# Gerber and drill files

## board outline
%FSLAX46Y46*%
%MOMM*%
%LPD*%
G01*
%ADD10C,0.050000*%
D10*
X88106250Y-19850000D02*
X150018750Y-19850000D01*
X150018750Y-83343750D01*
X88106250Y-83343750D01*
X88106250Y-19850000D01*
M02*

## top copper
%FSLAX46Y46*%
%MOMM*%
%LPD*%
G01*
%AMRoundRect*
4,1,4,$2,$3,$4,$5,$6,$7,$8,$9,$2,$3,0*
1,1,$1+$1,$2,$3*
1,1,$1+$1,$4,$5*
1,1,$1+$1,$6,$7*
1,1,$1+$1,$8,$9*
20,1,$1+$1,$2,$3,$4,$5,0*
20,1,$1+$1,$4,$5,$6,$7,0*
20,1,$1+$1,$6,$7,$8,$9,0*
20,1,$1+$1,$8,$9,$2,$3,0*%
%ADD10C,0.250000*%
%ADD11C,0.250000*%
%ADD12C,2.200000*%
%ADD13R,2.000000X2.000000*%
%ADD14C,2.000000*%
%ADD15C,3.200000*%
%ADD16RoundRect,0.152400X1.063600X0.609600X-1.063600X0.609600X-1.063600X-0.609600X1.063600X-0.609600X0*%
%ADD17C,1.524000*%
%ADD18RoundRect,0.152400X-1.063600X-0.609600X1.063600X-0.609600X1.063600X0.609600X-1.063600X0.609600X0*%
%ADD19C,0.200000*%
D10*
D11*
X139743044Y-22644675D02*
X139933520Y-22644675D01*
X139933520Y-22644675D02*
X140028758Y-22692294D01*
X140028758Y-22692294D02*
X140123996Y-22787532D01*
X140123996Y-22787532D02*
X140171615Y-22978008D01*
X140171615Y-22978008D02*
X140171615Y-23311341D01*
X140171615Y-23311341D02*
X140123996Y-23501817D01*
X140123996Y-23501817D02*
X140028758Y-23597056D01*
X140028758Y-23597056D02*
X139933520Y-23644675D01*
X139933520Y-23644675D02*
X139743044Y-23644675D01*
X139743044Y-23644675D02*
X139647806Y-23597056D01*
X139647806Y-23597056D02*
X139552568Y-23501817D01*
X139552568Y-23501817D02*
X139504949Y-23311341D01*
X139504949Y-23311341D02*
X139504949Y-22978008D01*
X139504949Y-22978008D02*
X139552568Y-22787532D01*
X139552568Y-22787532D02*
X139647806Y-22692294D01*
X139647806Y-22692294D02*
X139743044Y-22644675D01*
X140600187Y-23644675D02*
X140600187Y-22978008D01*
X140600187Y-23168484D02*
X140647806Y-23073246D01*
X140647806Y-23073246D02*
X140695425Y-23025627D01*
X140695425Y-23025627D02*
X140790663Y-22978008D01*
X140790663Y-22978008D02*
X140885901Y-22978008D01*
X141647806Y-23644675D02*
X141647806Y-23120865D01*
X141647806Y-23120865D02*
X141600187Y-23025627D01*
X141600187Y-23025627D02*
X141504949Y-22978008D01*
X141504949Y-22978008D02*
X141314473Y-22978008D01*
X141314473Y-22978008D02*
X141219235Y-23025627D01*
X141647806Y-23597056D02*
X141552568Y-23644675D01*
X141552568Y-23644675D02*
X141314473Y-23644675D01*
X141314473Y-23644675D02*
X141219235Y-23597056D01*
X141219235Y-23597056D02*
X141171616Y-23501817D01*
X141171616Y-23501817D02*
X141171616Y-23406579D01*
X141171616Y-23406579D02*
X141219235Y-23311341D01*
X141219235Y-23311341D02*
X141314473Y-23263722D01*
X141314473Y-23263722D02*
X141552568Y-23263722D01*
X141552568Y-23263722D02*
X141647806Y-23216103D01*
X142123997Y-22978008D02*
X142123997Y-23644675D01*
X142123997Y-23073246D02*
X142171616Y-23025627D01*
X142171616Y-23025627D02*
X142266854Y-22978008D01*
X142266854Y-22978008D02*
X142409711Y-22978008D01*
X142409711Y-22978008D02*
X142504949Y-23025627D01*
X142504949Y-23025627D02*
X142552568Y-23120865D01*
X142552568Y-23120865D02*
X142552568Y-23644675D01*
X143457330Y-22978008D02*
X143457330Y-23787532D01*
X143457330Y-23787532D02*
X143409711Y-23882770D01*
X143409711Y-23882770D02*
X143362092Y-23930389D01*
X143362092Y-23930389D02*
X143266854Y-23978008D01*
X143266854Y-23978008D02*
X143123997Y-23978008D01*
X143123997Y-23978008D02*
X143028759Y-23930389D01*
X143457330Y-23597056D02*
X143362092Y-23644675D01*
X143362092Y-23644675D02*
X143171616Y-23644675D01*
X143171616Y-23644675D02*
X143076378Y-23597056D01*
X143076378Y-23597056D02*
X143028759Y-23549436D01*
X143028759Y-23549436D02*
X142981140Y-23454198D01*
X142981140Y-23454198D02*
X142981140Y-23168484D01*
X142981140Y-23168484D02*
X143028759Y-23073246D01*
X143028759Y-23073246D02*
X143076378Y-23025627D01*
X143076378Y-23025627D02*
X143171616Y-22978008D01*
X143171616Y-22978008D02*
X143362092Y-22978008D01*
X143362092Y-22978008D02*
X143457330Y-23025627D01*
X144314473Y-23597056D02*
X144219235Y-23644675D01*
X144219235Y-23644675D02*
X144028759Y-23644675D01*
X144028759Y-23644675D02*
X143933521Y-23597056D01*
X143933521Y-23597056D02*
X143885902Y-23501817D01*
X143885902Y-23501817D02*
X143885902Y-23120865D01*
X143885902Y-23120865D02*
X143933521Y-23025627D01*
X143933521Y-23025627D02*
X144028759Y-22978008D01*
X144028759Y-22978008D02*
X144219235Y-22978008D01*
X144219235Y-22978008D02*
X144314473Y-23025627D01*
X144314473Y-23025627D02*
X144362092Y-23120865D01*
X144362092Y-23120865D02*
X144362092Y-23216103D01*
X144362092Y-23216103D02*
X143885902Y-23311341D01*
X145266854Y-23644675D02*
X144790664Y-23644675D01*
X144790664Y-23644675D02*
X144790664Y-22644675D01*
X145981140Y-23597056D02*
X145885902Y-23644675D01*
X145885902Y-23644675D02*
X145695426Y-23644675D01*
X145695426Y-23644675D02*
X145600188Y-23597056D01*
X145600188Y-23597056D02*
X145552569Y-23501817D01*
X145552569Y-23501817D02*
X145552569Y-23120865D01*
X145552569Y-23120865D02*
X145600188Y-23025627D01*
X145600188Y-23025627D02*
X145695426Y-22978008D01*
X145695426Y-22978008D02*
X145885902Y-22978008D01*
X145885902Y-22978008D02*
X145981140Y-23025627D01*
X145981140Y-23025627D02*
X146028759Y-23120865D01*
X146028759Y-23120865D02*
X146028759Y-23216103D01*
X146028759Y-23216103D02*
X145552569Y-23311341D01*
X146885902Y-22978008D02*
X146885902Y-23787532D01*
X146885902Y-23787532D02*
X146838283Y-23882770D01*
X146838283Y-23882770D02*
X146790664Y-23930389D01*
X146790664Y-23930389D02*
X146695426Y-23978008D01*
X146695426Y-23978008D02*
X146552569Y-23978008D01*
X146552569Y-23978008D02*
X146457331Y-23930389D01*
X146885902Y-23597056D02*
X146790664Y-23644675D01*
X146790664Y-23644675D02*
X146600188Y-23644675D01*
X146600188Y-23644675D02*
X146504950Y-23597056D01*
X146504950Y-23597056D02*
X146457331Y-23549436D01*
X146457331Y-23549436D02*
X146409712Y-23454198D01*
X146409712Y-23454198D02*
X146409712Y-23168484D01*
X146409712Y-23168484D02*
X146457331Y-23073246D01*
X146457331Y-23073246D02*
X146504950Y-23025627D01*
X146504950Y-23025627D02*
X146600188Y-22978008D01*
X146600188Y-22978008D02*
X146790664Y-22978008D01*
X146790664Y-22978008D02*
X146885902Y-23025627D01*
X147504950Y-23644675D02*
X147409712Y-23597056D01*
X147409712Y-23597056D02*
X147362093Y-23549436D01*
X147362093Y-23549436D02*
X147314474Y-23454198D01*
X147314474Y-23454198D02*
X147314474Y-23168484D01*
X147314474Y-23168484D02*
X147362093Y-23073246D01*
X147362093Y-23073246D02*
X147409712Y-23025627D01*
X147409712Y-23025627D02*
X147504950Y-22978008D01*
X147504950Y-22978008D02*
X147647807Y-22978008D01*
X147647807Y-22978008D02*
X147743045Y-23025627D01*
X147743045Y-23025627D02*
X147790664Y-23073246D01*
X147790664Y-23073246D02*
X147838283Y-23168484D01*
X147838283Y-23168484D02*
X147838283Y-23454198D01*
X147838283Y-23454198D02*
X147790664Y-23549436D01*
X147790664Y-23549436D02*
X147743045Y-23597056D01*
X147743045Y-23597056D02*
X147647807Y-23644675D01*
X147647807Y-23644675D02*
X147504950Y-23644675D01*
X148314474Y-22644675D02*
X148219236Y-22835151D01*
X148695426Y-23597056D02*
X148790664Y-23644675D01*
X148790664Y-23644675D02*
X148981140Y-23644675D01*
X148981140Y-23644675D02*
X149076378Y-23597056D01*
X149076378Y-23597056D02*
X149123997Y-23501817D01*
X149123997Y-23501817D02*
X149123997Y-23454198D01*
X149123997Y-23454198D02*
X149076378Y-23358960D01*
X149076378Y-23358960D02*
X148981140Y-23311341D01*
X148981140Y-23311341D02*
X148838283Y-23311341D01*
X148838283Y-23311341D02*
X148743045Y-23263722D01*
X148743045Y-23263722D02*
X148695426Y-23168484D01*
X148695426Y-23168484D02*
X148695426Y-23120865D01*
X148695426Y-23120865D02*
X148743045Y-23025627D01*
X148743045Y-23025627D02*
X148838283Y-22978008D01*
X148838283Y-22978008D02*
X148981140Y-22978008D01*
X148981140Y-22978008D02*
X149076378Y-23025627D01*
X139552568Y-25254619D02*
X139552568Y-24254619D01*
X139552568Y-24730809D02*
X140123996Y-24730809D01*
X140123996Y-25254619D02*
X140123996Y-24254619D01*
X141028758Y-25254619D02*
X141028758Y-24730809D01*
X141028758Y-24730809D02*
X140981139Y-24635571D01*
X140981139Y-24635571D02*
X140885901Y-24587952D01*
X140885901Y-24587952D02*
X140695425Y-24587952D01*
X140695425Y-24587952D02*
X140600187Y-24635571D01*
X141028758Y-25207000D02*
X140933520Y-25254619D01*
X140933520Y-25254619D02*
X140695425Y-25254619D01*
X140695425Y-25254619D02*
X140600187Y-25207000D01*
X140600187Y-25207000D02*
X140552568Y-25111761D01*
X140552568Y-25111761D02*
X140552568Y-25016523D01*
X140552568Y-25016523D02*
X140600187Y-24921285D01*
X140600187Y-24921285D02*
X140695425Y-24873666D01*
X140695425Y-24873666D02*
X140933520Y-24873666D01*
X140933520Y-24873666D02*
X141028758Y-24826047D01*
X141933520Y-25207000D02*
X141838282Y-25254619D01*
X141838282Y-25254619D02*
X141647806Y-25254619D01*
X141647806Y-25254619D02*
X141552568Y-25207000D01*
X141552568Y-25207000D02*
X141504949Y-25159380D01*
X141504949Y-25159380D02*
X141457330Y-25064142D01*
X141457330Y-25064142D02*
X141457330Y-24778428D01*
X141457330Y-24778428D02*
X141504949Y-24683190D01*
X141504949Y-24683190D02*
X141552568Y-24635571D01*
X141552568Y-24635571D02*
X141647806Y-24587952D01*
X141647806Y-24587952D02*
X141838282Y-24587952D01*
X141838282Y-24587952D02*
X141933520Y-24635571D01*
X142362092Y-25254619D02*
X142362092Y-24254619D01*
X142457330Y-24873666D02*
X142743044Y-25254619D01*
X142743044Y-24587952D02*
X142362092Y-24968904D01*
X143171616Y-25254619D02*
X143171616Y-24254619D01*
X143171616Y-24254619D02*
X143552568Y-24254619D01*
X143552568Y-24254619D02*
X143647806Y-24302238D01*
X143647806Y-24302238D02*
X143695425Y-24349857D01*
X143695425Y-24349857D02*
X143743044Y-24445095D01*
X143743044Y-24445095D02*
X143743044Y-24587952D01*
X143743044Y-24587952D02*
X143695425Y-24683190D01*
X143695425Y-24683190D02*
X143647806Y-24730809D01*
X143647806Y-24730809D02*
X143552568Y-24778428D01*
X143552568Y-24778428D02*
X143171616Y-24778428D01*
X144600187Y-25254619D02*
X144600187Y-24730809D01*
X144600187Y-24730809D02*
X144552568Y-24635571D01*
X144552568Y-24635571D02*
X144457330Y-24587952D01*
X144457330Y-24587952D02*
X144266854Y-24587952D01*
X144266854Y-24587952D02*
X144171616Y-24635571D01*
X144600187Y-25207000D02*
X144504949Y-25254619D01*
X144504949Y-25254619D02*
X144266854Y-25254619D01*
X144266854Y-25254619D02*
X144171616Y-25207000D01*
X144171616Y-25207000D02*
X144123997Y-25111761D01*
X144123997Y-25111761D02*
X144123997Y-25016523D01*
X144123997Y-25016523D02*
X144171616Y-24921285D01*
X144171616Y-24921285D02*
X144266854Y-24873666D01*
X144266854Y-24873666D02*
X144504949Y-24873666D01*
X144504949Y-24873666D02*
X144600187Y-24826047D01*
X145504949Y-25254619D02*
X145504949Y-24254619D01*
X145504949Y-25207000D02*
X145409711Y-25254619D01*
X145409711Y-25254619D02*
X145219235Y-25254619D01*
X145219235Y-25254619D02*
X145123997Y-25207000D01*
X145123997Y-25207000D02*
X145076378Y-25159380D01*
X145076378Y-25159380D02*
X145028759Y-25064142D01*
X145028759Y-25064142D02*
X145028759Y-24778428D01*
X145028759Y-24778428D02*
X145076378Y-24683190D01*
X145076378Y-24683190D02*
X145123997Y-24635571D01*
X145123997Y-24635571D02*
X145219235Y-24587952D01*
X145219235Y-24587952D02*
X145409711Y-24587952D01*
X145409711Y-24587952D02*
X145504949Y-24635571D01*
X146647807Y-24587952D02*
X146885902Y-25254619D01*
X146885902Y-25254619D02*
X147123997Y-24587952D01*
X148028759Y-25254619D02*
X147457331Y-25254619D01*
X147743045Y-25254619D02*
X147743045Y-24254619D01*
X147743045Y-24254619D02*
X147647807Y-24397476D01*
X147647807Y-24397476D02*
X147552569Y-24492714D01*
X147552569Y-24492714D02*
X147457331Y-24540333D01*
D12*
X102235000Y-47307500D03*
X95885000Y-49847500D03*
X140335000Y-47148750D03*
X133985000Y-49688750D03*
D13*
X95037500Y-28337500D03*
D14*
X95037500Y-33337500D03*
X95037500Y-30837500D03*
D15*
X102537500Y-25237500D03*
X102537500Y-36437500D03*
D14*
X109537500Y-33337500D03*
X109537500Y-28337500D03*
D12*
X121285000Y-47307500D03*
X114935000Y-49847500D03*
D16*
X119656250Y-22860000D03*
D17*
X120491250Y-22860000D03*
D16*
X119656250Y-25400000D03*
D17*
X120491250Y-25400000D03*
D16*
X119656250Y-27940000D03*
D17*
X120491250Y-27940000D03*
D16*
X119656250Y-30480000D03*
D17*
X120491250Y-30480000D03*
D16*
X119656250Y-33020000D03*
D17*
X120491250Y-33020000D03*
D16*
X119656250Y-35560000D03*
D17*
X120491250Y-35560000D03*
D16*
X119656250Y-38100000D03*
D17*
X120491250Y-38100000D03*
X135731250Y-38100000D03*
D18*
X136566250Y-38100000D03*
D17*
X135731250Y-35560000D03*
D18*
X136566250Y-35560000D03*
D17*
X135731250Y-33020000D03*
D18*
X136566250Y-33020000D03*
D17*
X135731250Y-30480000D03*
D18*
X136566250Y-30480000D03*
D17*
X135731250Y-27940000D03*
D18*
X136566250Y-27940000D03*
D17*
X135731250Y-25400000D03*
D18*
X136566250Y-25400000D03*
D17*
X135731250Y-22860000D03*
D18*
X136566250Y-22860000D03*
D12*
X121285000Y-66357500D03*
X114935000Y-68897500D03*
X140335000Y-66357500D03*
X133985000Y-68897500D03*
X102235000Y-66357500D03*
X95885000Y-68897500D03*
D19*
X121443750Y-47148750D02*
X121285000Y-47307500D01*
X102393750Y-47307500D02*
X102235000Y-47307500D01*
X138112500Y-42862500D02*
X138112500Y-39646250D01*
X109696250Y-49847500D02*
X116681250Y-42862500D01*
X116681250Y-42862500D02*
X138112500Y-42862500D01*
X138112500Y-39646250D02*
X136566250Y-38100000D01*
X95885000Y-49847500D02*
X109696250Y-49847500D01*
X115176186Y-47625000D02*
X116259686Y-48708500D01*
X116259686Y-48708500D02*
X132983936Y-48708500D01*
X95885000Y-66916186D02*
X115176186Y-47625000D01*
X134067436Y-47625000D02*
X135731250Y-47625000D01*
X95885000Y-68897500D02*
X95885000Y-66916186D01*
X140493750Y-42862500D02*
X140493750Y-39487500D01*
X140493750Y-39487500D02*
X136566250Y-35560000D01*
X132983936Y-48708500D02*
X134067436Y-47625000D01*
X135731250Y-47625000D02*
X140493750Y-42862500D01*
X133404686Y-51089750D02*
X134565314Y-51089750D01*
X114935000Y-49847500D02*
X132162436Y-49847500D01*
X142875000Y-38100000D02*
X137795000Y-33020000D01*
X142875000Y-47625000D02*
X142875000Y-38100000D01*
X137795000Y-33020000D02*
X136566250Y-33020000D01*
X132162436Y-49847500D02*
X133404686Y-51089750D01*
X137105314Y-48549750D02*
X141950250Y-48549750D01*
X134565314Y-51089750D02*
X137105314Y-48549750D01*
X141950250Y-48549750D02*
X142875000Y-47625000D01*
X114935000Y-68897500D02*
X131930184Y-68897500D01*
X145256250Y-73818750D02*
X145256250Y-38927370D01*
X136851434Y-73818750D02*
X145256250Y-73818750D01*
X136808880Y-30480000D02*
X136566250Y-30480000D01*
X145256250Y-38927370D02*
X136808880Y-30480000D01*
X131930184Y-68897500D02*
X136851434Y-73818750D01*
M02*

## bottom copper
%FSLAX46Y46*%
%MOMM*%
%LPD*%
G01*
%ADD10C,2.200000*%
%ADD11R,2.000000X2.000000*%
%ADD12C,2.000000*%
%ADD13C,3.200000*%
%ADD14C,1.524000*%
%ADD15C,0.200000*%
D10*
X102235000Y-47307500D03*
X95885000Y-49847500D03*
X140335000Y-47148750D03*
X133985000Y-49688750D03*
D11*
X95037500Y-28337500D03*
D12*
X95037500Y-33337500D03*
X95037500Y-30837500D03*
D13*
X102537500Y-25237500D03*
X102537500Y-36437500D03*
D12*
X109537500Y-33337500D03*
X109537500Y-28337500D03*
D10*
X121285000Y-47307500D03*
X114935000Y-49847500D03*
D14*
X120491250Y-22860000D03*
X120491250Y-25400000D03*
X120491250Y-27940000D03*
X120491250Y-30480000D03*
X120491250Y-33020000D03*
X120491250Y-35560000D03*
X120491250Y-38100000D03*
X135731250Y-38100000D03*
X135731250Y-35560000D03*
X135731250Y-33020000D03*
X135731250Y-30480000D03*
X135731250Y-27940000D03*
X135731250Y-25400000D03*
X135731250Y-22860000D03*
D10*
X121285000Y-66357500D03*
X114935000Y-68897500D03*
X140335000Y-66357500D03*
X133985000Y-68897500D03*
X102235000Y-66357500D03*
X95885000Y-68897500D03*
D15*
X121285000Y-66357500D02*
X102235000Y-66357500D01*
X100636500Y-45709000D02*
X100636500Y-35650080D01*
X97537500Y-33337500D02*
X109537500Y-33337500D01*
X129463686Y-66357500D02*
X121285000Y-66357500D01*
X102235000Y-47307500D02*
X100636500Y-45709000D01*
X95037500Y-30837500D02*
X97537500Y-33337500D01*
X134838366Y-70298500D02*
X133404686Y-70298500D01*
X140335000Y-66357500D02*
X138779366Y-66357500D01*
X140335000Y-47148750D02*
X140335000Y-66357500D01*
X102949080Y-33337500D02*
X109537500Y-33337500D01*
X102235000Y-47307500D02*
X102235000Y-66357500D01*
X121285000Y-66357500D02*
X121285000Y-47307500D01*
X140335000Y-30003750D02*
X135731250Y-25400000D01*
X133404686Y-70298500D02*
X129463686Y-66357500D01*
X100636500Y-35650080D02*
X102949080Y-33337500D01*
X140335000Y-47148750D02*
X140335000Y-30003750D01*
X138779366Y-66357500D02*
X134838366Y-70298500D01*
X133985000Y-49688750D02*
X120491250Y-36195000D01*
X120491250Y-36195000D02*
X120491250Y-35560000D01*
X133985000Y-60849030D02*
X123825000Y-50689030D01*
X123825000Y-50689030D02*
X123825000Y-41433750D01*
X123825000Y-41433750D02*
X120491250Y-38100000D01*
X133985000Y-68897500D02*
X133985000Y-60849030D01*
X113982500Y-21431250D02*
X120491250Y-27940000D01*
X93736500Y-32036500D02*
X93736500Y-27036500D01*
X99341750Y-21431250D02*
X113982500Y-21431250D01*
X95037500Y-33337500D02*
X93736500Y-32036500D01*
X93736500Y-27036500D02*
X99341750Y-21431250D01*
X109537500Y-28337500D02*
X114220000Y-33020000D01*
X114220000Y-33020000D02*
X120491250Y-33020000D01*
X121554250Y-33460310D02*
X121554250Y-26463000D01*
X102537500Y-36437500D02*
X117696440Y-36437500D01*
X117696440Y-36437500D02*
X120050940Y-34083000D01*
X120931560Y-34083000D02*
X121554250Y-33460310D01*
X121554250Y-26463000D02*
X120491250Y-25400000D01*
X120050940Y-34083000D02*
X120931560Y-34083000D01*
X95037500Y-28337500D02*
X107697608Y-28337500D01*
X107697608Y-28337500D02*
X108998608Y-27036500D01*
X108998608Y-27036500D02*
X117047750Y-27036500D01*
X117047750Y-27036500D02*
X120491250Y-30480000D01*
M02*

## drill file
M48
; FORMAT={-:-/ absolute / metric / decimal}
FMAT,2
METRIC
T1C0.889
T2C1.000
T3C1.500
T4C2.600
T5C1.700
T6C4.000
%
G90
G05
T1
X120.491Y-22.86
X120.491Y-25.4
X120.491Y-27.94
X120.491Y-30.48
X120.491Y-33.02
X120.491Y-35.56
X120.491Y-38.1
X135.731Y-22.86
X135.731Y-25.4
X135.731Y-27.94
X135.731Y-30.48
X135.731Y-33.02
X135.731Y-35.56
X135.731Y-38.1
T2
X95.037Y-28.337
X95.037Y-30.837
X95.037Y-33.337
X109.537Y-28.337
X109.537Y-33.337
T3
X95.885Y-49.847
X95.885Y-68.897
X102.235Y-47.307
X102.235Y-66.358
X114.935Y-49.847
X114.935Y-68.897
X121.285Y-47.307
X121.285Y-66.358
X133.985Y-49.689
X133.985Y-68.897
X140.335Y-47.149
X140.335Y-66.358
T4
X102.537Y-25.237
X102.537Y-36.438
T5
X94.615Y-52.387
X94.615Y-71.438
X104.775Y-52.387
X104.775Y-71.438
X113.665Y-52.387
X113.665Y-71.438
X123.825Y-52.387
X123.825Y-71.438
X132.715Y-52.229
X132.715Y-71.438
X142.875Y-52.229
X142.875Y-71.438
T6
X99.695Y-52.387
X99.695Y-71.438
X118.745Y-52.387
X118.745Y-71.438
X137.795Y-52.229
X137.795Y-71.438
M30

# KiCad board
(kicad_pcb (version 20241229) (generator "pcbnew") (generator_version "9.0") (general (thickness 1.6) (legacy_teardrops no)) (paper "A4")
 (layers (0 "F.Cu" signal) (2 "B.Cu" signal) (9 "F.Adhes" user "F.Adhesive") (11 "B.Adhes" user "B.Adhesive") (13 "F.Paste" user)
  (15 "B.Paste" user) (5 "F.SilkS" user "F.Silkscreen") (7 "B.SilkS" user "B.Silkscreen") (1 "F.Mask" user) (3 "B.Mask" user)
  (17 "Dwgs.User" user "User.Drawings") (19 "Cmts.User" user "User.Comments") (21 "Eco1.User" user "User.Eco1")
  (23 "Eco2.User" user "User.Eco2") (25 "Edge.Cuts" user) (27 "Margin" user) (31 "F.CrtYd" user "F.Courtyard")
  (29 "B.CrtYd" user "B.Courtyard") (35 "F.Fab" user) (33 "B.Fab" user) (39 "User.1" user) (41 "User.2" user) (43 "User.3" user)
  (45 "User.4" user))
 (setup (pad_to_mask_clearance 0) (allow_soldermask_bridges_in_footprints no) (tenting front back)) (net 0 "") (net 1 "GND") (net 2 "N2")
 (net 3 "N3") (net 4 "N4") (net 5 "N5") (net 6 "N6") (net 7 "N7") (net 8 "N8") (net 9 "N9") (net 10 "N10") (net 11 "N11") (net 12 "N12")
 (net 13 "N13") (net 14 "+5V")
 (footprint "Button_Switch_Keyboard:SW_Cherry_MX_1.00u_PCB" (layer "F.Cu") (at 102.235 47.3075)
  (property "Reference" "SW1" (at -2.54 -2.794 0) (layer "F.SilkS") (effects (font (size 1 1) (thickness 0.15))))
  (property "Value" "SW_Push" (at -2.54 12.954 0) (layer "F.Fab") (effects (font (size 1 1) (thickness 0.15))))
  (pad "" np_thru_hole circle (at -7.62 5.08) (size 1.7 1.7) (drill 1.7) (layers "*.Cu" "*.Mask"))
  (pad "" np_thru_hole circle (at -2.54 5.08) (size 4 4) (drill 4) (layers "*.Cu" "*.Mask"))
  (pad "" np_thru_hole circle (at 2.54 5.08) (size 1.7 1.7) (drill 1.7) (layers "*.Cu" "*.Mask"))
  (pad "1" thru_hole circle (at 0 0) (size 2.2 2.2) (drill 1.5) (layers "*.Cu" "*.Mask") (remove_unused_layers no) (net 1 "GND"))
  (pad "2" thru_hole circle (at -6.35 2.54) (size 2.2 2.2) (drill 1.5) (layers "*.Cu" "*.Mask") (remove_unused_layers no) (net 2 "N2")))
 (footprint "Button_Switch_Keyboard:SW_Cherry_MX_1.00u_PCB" (layer "F.Cu") (at 140.335 47.14875)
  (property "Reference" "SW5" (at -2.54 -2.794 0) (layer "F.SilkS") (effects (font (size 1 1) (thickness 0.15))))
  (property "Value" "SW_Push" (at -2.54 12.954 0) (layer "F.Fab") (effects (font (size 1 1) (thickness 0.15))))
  (pad "" np_thru_hole circle (at -7.62 5.08) (size 1.7 1.7) (drill 1.7) (layers "*.Cu" "*.Mask"))
  (pad "" np_thru_hole circle (at -2.54 5.08) (size 4 4) (drill 4) (layers "*.Cu" "*.Mask"))
  (pad "" np_thru_hole circle (at 2.54 5.08) (size 1.7 1.7) (drill 1.7) (layers "*.Cu" "*.Mask"))
  (pad "1" thru_hole circle (at 0 0) (size 2.2 2.2) (drill 1.5) (layers "*.Cu" "*.Mask") (remove_unused_layers no) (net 1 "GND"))
  (pad "2" thru_hole circle (at -6.35 2.54) (size 2.2 2.2) (drill 1.5) (layers "*.Cu" "*.Mask") (remove_unused_layers no) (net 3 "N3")))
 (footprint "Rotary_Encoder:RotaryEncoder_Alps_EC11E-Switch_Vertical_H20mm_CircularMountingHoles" (layer "F.Cu") (at 95.0375 28.3375)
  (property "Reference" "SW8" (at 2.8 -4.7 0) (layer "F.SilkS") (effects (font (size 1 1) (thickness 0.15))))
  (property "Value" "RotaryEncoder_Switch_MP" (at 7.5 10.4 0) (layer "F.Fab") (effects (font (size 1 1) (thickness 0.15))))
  (pad "A" thru_hole rect (at 0 0) (size 2 2) (drill 1) (layers "*.Cu" "*.Mask") (remove_unused_layers no) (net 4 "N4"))
  (pad "B" thru_hole circle (at 0 5) (size 2 2) (drill 1) (layers "*.Cu" "*.Mask") (remove_unused_layers no) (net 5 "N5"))
  (pad "C" thru_hole circle (at 0 2.5) (size 2 2) (drill 1) (layers "*.Cu" "*.Mask") (remove_unused_layers no) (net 1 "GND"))
  (pad "MP" thru_hole circle (at 7.5 -3.1) (size 3.2 3.2) (drill 2.6) (layers "*.Cu" "*.Mask") (remove_unused_layers no) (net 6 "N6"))
  (pad "MP" thru_hole circle (at 7.5 8.1) (size 3.2 3.2) (drill 2.6) (layers "*.Cu" "*.Mask") (remove_unused_layers no) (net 6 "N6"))
  (pad "S1" thru_hole circle (at 14.5 5) (size 2 2) (drill 1) (layers "*.Cu" "*.Mask") (remove_unused_layers no) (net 1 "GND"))
  (pad "S2" thru_hole circle (at 14.5 0) (size 2 2) (drill 1) (layers "*.Cu" "*.Mask") (remove_unused_layers no) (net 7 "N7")))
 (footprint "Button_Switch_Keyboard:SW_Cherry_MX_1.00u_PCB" (layer "F.Cu") (at 121.285 47.3075)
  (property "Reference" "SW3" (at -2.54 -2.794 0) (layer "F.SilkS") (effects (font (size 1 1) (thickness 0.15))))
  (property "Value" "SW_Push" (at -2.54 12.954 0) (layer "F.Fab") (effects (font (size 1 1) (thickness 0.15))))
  (pad "" np_thru_hole circle (at -7.62 5.08) (size 1.7 1.7) (drill 1.7) (layers "*.Cu" "*.Mask"))
  (pad "" np_thru_hole circle (at -2.54 5.08) (size 4 4) (drill 4) (layers "*.Cu" "*.Mask"))
  (pad "" np_thru_hole circle (at 2.54 5.08) (size 1.7 1.7) (drill 1.7) (layers "*.Cu" "*.Mask"))
  (pad "1" thru_hole circle (at 0 0) (size 2.2 2.2) (drill 1.5) (layers "*.Cu" "*.Mask") (remove_unused_layers no) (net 1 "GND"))
  (pad "2" thru_hole circle (at -6.35 2.54) (size 2.2 2.2) (drill 1.5) (layers "*.Cu" "*.Mask") (remove_unused_layers no) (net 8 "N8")))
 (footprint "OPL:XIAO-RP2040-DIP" (layer "F.Cu") (at 128.11125 30.48)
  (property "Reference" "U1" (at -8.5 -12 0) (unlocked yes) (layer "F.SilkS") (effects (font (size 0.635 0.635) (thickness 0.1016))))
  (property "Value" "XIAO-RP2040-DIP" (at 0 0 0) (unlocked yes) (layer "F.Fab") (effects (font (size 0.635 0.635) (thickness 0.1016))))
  (pad "1" smd roundrect (at -8.455 -7.62 180) (size 2.432 1.524) (layers "F.Cu" "F.Mask") (roundrect_rratio 0.1) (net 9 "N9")
   (thermal_bridge_angle 45))
  (pad "1" thru_hole circle (at -7.62 -7.62 180) (size 1.524 1.524) (drill 0.889) (layers "*.Cu" "*.Mask") (remove_unused_layers no)
   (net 9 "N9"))
  (pad "2" smd roundrect (at -8.455 -5.08 180) (size 2.432 1.524) (layers "F.Cu" "F.Mask") (roundrect_rratio 0.1) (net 6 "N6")
   (thermal_bridge_angle 45))
  (pad "2" thru_hole circle (at -7.62 -5.08 180) (size 1.524 1.524) (drill 0.889) (layers "*.Cu" "*.Mask") (remove_unused_layers no)
   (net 6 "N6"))
  (pad "3" smd roundrect (at -8.455 -2.54 180) (size 2.432 1.524) (layers "F.Cu" "F.Mask") (roundrect_rratio 0.1) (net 5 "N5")
   (thermal_bridge_angle 45))
  (pad "3" thru_hole circle (at -7.62 -2.54 180) (size 1.524 1.524) (drill 0.889) (layers "*.Cu" "*.Mask") (remove_unused_layers no)
   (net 5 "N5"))
  (pad "4" smd roundrect (at -8.455 0 180) (size 2.432 1.524) (layers "F.Cu" "F.Mask") (roundrect_rratio 0.1) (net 4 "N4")
   (thermal_bridge_angle 45))
  (pad "4" thru_hole circle (at -7.62 0 180) (size 1.524 1.524) (drill 0.889) (layers "*.Cu" "*.Mask") (remove_unused_layers no)
   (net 4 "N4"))
  (pad "5" smd roundrect (at -8.455 2.54 180) (size 2.432 1.524) (layers "F.Cu" "F.Mask") (roundrect_rratio 0.1) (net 7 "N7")
   (thermal_bridge_angle 45))
  (pad "5" thru_hole circle (at -7.62 2.54 180) (size 1.524 1.524) (drill 0.889) (layers "*.Cu" "*.Mask") (remove_unused_layers no)
   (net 7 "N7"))
  (pad "6" smd roundrect (at -8.455 5.08 180) (size 2.432 1.524) (layers "F.Cu" "F.Mask") (roundrect_rratio 0.1) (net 3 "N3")
   (thermal_bridge_angle 45))
  (pad "6" thru_hole circle (at -7.62 5.08 180) (size 1.524 1.524) (drill 0.889) (layers "*.Cu" "*.Mask") (remove_unused_layers no)
   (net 3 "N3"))
  (pad "7" smd roundrect (at -8.455 7.62 180) (size 2.432 1.524) (layers "F.Cu" "F.Mask") (roundrect_rratio 0.1) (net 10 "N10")
   (thermal_bridge_angle 45))
  (pad "7" thru_hole circle (at -7.62 7.62 180) (size 1.524 1.524) (drill 0.889) (layers "*.Cu" "*.Mask") (remove_unused_layers no)
   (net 10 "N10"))
  (pad "8" thru_hole circle (at 7.62 7.62) (size 1.524 1.524) (drill 0.889) (layers "*.Cu" "*.Mask") (remove_unused_layers no) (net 2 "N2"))
  (pad "8" smd roundrect (at 8.455 7.62) (size 2.432 1.524) (layers "F.Cu" "F.Mask") (roundrect_rratio 0.1) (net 2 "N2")
   (thermal_bridge_angle 45))
  (pad "9" thru_hole circle (at 7.62 5.08) (size 1.524 1.524) (drill 0.889) (layers "*.Cu" "*.Mask") (remove_unused_layers no)
   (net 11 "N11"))
  (pad "9" smd roundrect (at 8.455 5.08) (size 2.432 1.524) (layers "F.Cu" "F.Mask") (roundrect_rratio 0.1) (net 11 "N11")
   (thermal_bridge_angle 45))
  (pad "10" thru_hole circle (at 7.62 2.54) (size 1.524 1.524) (drill 0.889) (layers "*.Cu" "*.Mask") (remove_unused_layers no) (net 8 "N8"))
  (pad "10" smd roundrect (at 8.455 2.54) (size 2.432 1.524) (layers "F.Cu" "F.Mask") (roundrect_rratio 0.1) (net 8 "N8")
   (thermal_bridge_angle 45))
  (pad "11" thru_hole circle (at 7.62 0) (size 1.524 1.524) (drill 0.889) (layers "*.Cu" "*.Mask") (remove_unused_layers no) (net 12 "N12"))
  (pad "11" smd roundrect (at 8.455 0) (size 2.432 1.524) (layers "F.Cu" "F.Mask") (roundrect_rratio 0.1) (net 12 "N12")
   (thermal_bridge_angle 45))
  (pad "12" thru_hole circle (at 7.62 -2.54) (size 1.524 1.524) (drill 0.889) (layers "*.Cu" "*.Mask") (remove_unused_layers no)
   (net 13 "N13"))
  (pad "12" smd roundrect (at 8.455 -2.54) (size 2.432 1.524) (layers "F.Cu" "F.Mask") (roundrect_rratio 0.1) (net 13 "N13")
   (thermal_bridge_angle 45))
  (pad "13" thru_hole circle (at 7.62 -5.08) (size 1.524 1.524) (drill 0.889) (layers "*.Cu" "*.Mask") (remove_unused_layers no)
   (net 1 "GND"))
  (pad "13" smd roundrect (at 8.455 -5.08) (size 2.432 1.524) (layers "F.Cu" "F.Mask") (roundrect_rratio 0.1) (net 1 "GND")
   (thermal_bridge_angle 45))
  (pad "14" thru_hole circle (at 7.62 -7.62) (size 1.524 1.524) (drill 0.889) (layers "*.Cu" "*.Mask") (remove_unused_layers no)
   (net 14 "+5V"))
  (pad "14" smd roundrect (at 8.455 -7.62) (size 2.432 1.524) (layers "F.Cu" "F.Mask") (roundrect_rratio 0.1) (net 14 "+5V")
   (thermal_bridge_angle 45)))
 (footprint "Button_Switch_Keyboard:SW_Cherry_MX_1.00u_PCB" (layer "F.Cu") (at 121.285 66.3575)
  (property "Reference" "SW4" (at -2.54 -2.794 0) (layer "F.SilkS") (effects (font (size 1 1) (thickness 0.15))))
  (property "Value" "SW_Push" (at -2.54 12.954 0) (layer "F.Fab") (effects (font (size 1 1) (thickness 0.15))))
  (pad "" np_thru_hole circle (at -7.62 5.08) (size 1.7 1.7) (drill 1.7) (layers "*.Cu" "*.Mask"))
  (pad "" np_thru_hole circle (at -2.54 5.08) (size 4 4) (drill 4) (layers "*.Cu" "*.Mask"))
  (pad "" np_thru_hole circle (at 2.54 5.08) (size 1.7 1.7) (drill 1.7) (layers "*.Cu" "*.Mask"))
  (pad "1" thru_hole circle (at 0 0) (size 2.2 2.2) (drill 1.5) (layers "*.Cu" "*.Mask") (remove_unused_layers no) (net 1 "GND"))
  (pad "2" thru_hole circle (at -6.35 2.54) (size 2.2 2.2) (drill 1.5) (layers "*.Cu" "*.Mask") (remove_unused_layers no) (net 12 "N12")))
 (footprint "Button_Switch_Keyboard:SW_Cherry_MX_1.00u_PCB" (layer "F.Cu") (at 140.335 66.3575)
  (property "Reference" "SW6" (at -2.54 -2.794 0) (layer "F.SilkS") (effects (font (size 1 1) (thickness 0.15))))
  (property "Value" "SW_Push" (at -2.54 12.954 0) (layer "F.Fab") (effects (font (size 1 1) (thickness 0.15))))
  (pad "" np_thru_hole circle (at -7.62 5.08) (size 1.7 1.7) (drill 1.7) (layers "*.Cu" "*.Mask"))
  (pad "" np_thru_hole circle (at -2.54 5.08) (size 4 4) (drill 4) (layers "*.Cu" "*.Mask"))
  (pad "" np_thru_hole circle (at 2.54 5.08) (size 1.7 1.7) (drill 1.7) (layers "*.Cu" "*.Mask"))
  (pad "1" thru_hole circle (at 0 0) (size 2.2 2.2) (drill 1.5) (layers "*.Cu" "*.Mask") (remove_unused_layers no) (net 1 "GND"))
  (pad "2" thru_hole circle (at -6.35 2.54) (size 2.2 2.2) (drill 1.5) (layers "*.Cu" "*.Mask") (remove_unused_layers no) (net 10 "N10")))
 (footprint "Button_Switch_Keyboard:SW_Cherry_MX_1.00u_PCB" (layer "F.Cu") (at 102.235 66.3575)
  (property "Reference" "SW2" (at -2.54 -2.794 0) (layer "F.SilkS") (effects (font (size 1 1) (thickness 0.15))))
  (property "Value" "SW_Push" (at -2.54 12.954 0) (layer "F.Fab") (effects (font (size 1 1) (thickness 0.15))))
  (pad "" np_thru_hole circle (at -7.62 5.08) (size 1.7 1.7) (drill 1.7) (layers "*.Cu" "*.Mask"))
  (pad "" np_thru_hole circle (at -2.54 5.08) (size 4 4) (drill 4) (layers "*.Cu" "*.Mask"))
  (pad "" np_thru_hole circle (at 2.54 5.08) (size 1.7 1.7) (drill 1.7) (layers "*.Cu" "*.Mask"))
  (pad "1" thru_hole circle (at 0 0) (size 2.2 2.2) (drill 1.5) (layers "*.Cu" "*.Mask") (remove_unused_layers no) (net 1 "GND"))
  (pad "2" thru_hole circle (at -6.35 2.54) (size 2.2 2.2) (drill 1.5) (layers "*.Cu" "*.Mask") (remove_unused_layers no) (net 11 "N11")))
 (gr_rect (start 88.10625 19.85) (end 150.01875 83.34375) (stroke (width 0.05) (type default)) (fill no) (layer "Edge.Cuts"))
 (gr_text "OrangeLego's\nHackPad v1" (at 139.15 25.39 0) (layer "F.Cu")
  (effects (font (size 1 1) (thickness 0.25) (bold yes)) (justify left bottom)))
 (segment (start 121.44375 47.14875) (end 121.285 47.3075) (width 0.2) (layer "F.Cu") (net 1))
 (segment (start 102.39375 47.3075) (end 102.235 47.3075) (width 0.2) (layer "F.Cu") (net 1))
 (segment (start 121.285 66.3575) (end 102.235 66.3575) (width 0.2) (layer "B.Cu") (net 1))
 (segment (start 100.6365 45.709) (end 100.6365 35.65008) (width 0.2) (layer "B.Cu") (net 1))
 (segment (start 97.5375 33.3375) (end 109.5375 33.3375) (width 0.2) (layer "B.Cu") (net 1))
 (segment (start 129.463686 66.3575) (end 121.285 66.3575) (width 0.2) (layer "B.Cu") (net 1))
 (segment (start 102.235 47.3075) (end 100.6365 45.709) (width 0.2) (layer "B.Cu") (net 1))
 (segment (start 95.0375 30.8375) (end 97.5375 33.3375) (width 0.2) (layer "B.Cu") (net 1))
 (segment (start 134.838366 70.2985) (end 133.404686 70.2985) (width 0.2) (layer "B.Cu") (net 1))
 (segment (start 140.335 66.3575) (end 138.779366 66.3575) (width 0.2) (layer "B.Cu") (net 1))
 (segment (start 140.335 47.14875) (end 140.335 66.3575) (width 0.2) (layer "B.Cu") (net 1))
 (segment (start 102.94908 33.3375) (end 109.5375 33.3375) (width 0.2) (layer "B.Cu") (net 1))
 (segment (start 102.235 47.3075) (end 102.235 66.3575) (width 0.2) (layer "B.Cu") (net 1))
 (segment (start 121.285 66.3575) (end 121.285 47.3075) (width 0.2) (layer "B.Cu") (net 1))
 (segment (start 140.335 30.00375) (end 135.73125 25.4) (width 0.2) (layer "B.Cu") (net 1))
 (segment (start 133.404686 70.2985) (end 129.463686 66.3575) (width 0.2) (layer "B.Cu") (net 1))
 (segment (start 100.6365 35.65008) (end 102.94908 33.3375) (width 0.2) (layer "B.Cu") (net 1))
 (segment (start 140.335 47.14875) (end 140.335 30.00375) (width 0.2) (layer "B.Cu") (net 1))
 (segment (start 138.779366 66.3575) (end 134.838366 70.2985) (width 0.2) (layer "B.Cu") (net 1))
 (segment (start 138.1125 42.8625) (end 138.1125 39.64625) (width 0.2) (layer "F.Cu") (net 2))
 (segment (start 109.69625 49.8475) (end 116.68125 42.8625) (width 0.2) (layer "F.Cu") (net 2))
 (segment (start 116.68125 42.8625) (end 138.1125 42.8625) (width 0.2) (layer "F.Cu") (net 2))
 (segment (start 138.1125 39.64625) (end 136.56625 38.1) (width 0.2) (layer "F.Cu") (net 2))
 (segment (start 95.885 49.8475) (end 109.69625 49.8475) (width 0.2) (layer "F.Cu") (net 2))
 (segment (start 115.176186 47.625) (end 116.259686 48.7085) (width 0.2) (layer "F.Cu") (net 11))
 (segment (start 116.259686 48.7085) (end 132.983936 48.7085) (width 0.2) (layer "F.Cu") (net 11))
 (segment (start 95.885 66.916186) (end 115.176186 47.625) (width 0.2) (layer "F.Cu") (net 11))
 (segment (start 134.067436 47.625) (end 135.73125 47.625) (width 0.2) (layer "F.Cu") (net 11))
 (segment (start 95.885 68.8975) (end 95.885 66.916186) (width 0.2) (layer "F.Cu") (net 11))
 (segment (start 140.49375 42.8625) (end 140.49375 39.4875) (width 0.2) (layer "F.Cu") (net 11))
 (segment (start 140.49375 39.4875) (end 136.56625 35.56) (width 0.2) (layer "F.Cu") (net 11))
 (segment (start 132.983936 48.7085) (end 134.067436 47.625) (width 0.2) (layer "F.Cu") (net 11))
 (segment (start 135.73125 47.625) (end 140.49375 42.8625) (width 0.2) (layer "F.Cu") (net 11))
 (segment (start 133.404686 51.08975) (end 134.565314 51.08975) (width 0.2) (layer "F.Cu") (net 8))
 (segment (start 114.935 49.8475) (end 132.162436 49.8475) (width 0.2) (layer "F.Cu") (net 8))
 (segment (start 142.875 38.1) (end 137.795 33.02) (width 0.2) (layer "F.Cu") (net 8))
 (segment (start 142.875 47.625) (end 142.875 38.1) (width 0.2) (layer "F.Cu") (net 8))
 (segment (start 137.795 33.02) (end 136.56625 33.02) (width 0.2) (layer "F.Cu") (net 8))
 (segment (start 132.162436 49.8475) (end 133.404686 51.08975) (width 0.2) (layer "F.Cu") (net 8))
 (segment (start 137.105314 48.54975) (end 141.95025 48.54975) (width 0.2) (layer "F.Cu") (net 8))
 (segment (start 134.565314 51.08975) (end 137.105314 48.54975) (width 0.2) (layer "F.Cu") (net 8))
 (segment (start 141.95025 48.54975) (end 142.875 47.625) (width 0.2) (layer "F.Cu") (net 8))
 (segment (start 114.935 68.8975) (end 131.930184 68.8975) (width 0.2) (layer "F.Cu") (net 12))
 (segment (start 145.25625 73.81875) (end 145.25625 38.92737) (width 0.2) (layer "F.Cu") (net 12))
 (segment (start 136.851434 73.81875) (end 145.25625 73.81875) (width 0.2) (layer "F.Cu") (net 12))
 (segment (start 136.80888 30.48) (end 136.56625 30.48) (width 0.2) (layer "F.Cu") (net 12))
 (segment (start 145.25625 38.92737) (end 136.80888 30.48) (width 0.2) (layer "F.Cu") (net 12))
 (segment (start 131.930184 68.8975) (end 136.851434 73.81875) (width 0.2) (layer "F.Cu") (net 12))
 (segment (start 133.985 49.68875) (end 120.49125 36.195) (width 0.2) (layer "B.Cu") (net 3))
 (segment (start 120.49125 36.195) (end 120.49125 35.56) (width 0.2) (layer "B.Cu") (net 3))
 (segment (start 133.985 60.84903) (end 123.825 50.68903) (width 0.2) (layer "B.Cu") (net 10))
 (segment (start 123.825 50.68903) (end 123.825 41.43375) (width 0.2) (layer "B.Cu") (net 10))
 (segment (start 123.825 41.43375) (end 120.49125 38.1) (width 0.2) (layer "B.Cu") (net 10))
 (segment (start 133.985 68.8975) (end 133.985 60.84903) (width 0.2) (layer "B.Cu") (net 10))
 (segment (start 113.9825 21.43125) (end 120.49125 27.94) (width 0.2) (layer "B.Cu") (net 5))
 (segment (start 93.7365 32.0365) (end 93.7365 27.0365) (width 0.2) (layer "B.Cu") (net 5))
 (segment (start 99.34175 21.43125) (end 113.9825 21.43125) (width 0.2) (layer "B.Cu") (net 5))
 (segment (start 95.0375 33.3375) (end 93.7365 32.0365) (width 0.2) (layer "B.Cu") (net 5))
 (segment (start 93.7365 27.0365) (end 99.34175 21.43125) (width 0.2) (layer "B.Cu") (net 5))
 (segment (start 109.5375 28.3375) (end 114.22 33.02) (width 0.2) (layer "B.Cu") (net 7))
 (segment (start 114.22 33.02) (end 120.49125 33.02) (width 0.2) (layer "B.Cu") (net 7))
 (segment (start 121.55425 33.46031) (end 121.55425 26.463) (width 0.2) (layer "B.Cu") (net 6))
 (segment (start 102.5375 36.4375) (end 117.69644 36.4375) (width 0.2) (layer "B.Cu") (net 6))
 (segment (start 117.69644 36.4375) (end 120.05094 34.083) (width 0.2) (layer "B.Cu") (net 6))
 (segment (start 120.93156 34.083) (end 121.55425 33.46031) (width 0.2) (layer "B.Cu") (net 6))
 (segment (start 121.55425 26.463) (end 120.49125 25.4) (width 0.2) (layer "B.Cu") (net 6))
 (segment (start 120.05094 34.083) (end 120.93156 34.083) (width 0.2) (layer "B.Cu") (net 6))
 (segment (start 95.0375 28.3375) (end 107.697608 28.3375) (width 0.2) (layer "B.Cu") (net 4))
 (segment (start 107.697608 28.3375) (end 108.998608 27.0365) (width 0.2) (layer "B.Cu") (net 4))
 (segment (start 108.998608 27.0365) (end 117.04775 27.0365) (width 0.2) (layer "B.Cu") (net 4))
 (segment (start 117.04775 27.0365) (end 120.49125 30.48) (width 0.2) (layer "B.Cu") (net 4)))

